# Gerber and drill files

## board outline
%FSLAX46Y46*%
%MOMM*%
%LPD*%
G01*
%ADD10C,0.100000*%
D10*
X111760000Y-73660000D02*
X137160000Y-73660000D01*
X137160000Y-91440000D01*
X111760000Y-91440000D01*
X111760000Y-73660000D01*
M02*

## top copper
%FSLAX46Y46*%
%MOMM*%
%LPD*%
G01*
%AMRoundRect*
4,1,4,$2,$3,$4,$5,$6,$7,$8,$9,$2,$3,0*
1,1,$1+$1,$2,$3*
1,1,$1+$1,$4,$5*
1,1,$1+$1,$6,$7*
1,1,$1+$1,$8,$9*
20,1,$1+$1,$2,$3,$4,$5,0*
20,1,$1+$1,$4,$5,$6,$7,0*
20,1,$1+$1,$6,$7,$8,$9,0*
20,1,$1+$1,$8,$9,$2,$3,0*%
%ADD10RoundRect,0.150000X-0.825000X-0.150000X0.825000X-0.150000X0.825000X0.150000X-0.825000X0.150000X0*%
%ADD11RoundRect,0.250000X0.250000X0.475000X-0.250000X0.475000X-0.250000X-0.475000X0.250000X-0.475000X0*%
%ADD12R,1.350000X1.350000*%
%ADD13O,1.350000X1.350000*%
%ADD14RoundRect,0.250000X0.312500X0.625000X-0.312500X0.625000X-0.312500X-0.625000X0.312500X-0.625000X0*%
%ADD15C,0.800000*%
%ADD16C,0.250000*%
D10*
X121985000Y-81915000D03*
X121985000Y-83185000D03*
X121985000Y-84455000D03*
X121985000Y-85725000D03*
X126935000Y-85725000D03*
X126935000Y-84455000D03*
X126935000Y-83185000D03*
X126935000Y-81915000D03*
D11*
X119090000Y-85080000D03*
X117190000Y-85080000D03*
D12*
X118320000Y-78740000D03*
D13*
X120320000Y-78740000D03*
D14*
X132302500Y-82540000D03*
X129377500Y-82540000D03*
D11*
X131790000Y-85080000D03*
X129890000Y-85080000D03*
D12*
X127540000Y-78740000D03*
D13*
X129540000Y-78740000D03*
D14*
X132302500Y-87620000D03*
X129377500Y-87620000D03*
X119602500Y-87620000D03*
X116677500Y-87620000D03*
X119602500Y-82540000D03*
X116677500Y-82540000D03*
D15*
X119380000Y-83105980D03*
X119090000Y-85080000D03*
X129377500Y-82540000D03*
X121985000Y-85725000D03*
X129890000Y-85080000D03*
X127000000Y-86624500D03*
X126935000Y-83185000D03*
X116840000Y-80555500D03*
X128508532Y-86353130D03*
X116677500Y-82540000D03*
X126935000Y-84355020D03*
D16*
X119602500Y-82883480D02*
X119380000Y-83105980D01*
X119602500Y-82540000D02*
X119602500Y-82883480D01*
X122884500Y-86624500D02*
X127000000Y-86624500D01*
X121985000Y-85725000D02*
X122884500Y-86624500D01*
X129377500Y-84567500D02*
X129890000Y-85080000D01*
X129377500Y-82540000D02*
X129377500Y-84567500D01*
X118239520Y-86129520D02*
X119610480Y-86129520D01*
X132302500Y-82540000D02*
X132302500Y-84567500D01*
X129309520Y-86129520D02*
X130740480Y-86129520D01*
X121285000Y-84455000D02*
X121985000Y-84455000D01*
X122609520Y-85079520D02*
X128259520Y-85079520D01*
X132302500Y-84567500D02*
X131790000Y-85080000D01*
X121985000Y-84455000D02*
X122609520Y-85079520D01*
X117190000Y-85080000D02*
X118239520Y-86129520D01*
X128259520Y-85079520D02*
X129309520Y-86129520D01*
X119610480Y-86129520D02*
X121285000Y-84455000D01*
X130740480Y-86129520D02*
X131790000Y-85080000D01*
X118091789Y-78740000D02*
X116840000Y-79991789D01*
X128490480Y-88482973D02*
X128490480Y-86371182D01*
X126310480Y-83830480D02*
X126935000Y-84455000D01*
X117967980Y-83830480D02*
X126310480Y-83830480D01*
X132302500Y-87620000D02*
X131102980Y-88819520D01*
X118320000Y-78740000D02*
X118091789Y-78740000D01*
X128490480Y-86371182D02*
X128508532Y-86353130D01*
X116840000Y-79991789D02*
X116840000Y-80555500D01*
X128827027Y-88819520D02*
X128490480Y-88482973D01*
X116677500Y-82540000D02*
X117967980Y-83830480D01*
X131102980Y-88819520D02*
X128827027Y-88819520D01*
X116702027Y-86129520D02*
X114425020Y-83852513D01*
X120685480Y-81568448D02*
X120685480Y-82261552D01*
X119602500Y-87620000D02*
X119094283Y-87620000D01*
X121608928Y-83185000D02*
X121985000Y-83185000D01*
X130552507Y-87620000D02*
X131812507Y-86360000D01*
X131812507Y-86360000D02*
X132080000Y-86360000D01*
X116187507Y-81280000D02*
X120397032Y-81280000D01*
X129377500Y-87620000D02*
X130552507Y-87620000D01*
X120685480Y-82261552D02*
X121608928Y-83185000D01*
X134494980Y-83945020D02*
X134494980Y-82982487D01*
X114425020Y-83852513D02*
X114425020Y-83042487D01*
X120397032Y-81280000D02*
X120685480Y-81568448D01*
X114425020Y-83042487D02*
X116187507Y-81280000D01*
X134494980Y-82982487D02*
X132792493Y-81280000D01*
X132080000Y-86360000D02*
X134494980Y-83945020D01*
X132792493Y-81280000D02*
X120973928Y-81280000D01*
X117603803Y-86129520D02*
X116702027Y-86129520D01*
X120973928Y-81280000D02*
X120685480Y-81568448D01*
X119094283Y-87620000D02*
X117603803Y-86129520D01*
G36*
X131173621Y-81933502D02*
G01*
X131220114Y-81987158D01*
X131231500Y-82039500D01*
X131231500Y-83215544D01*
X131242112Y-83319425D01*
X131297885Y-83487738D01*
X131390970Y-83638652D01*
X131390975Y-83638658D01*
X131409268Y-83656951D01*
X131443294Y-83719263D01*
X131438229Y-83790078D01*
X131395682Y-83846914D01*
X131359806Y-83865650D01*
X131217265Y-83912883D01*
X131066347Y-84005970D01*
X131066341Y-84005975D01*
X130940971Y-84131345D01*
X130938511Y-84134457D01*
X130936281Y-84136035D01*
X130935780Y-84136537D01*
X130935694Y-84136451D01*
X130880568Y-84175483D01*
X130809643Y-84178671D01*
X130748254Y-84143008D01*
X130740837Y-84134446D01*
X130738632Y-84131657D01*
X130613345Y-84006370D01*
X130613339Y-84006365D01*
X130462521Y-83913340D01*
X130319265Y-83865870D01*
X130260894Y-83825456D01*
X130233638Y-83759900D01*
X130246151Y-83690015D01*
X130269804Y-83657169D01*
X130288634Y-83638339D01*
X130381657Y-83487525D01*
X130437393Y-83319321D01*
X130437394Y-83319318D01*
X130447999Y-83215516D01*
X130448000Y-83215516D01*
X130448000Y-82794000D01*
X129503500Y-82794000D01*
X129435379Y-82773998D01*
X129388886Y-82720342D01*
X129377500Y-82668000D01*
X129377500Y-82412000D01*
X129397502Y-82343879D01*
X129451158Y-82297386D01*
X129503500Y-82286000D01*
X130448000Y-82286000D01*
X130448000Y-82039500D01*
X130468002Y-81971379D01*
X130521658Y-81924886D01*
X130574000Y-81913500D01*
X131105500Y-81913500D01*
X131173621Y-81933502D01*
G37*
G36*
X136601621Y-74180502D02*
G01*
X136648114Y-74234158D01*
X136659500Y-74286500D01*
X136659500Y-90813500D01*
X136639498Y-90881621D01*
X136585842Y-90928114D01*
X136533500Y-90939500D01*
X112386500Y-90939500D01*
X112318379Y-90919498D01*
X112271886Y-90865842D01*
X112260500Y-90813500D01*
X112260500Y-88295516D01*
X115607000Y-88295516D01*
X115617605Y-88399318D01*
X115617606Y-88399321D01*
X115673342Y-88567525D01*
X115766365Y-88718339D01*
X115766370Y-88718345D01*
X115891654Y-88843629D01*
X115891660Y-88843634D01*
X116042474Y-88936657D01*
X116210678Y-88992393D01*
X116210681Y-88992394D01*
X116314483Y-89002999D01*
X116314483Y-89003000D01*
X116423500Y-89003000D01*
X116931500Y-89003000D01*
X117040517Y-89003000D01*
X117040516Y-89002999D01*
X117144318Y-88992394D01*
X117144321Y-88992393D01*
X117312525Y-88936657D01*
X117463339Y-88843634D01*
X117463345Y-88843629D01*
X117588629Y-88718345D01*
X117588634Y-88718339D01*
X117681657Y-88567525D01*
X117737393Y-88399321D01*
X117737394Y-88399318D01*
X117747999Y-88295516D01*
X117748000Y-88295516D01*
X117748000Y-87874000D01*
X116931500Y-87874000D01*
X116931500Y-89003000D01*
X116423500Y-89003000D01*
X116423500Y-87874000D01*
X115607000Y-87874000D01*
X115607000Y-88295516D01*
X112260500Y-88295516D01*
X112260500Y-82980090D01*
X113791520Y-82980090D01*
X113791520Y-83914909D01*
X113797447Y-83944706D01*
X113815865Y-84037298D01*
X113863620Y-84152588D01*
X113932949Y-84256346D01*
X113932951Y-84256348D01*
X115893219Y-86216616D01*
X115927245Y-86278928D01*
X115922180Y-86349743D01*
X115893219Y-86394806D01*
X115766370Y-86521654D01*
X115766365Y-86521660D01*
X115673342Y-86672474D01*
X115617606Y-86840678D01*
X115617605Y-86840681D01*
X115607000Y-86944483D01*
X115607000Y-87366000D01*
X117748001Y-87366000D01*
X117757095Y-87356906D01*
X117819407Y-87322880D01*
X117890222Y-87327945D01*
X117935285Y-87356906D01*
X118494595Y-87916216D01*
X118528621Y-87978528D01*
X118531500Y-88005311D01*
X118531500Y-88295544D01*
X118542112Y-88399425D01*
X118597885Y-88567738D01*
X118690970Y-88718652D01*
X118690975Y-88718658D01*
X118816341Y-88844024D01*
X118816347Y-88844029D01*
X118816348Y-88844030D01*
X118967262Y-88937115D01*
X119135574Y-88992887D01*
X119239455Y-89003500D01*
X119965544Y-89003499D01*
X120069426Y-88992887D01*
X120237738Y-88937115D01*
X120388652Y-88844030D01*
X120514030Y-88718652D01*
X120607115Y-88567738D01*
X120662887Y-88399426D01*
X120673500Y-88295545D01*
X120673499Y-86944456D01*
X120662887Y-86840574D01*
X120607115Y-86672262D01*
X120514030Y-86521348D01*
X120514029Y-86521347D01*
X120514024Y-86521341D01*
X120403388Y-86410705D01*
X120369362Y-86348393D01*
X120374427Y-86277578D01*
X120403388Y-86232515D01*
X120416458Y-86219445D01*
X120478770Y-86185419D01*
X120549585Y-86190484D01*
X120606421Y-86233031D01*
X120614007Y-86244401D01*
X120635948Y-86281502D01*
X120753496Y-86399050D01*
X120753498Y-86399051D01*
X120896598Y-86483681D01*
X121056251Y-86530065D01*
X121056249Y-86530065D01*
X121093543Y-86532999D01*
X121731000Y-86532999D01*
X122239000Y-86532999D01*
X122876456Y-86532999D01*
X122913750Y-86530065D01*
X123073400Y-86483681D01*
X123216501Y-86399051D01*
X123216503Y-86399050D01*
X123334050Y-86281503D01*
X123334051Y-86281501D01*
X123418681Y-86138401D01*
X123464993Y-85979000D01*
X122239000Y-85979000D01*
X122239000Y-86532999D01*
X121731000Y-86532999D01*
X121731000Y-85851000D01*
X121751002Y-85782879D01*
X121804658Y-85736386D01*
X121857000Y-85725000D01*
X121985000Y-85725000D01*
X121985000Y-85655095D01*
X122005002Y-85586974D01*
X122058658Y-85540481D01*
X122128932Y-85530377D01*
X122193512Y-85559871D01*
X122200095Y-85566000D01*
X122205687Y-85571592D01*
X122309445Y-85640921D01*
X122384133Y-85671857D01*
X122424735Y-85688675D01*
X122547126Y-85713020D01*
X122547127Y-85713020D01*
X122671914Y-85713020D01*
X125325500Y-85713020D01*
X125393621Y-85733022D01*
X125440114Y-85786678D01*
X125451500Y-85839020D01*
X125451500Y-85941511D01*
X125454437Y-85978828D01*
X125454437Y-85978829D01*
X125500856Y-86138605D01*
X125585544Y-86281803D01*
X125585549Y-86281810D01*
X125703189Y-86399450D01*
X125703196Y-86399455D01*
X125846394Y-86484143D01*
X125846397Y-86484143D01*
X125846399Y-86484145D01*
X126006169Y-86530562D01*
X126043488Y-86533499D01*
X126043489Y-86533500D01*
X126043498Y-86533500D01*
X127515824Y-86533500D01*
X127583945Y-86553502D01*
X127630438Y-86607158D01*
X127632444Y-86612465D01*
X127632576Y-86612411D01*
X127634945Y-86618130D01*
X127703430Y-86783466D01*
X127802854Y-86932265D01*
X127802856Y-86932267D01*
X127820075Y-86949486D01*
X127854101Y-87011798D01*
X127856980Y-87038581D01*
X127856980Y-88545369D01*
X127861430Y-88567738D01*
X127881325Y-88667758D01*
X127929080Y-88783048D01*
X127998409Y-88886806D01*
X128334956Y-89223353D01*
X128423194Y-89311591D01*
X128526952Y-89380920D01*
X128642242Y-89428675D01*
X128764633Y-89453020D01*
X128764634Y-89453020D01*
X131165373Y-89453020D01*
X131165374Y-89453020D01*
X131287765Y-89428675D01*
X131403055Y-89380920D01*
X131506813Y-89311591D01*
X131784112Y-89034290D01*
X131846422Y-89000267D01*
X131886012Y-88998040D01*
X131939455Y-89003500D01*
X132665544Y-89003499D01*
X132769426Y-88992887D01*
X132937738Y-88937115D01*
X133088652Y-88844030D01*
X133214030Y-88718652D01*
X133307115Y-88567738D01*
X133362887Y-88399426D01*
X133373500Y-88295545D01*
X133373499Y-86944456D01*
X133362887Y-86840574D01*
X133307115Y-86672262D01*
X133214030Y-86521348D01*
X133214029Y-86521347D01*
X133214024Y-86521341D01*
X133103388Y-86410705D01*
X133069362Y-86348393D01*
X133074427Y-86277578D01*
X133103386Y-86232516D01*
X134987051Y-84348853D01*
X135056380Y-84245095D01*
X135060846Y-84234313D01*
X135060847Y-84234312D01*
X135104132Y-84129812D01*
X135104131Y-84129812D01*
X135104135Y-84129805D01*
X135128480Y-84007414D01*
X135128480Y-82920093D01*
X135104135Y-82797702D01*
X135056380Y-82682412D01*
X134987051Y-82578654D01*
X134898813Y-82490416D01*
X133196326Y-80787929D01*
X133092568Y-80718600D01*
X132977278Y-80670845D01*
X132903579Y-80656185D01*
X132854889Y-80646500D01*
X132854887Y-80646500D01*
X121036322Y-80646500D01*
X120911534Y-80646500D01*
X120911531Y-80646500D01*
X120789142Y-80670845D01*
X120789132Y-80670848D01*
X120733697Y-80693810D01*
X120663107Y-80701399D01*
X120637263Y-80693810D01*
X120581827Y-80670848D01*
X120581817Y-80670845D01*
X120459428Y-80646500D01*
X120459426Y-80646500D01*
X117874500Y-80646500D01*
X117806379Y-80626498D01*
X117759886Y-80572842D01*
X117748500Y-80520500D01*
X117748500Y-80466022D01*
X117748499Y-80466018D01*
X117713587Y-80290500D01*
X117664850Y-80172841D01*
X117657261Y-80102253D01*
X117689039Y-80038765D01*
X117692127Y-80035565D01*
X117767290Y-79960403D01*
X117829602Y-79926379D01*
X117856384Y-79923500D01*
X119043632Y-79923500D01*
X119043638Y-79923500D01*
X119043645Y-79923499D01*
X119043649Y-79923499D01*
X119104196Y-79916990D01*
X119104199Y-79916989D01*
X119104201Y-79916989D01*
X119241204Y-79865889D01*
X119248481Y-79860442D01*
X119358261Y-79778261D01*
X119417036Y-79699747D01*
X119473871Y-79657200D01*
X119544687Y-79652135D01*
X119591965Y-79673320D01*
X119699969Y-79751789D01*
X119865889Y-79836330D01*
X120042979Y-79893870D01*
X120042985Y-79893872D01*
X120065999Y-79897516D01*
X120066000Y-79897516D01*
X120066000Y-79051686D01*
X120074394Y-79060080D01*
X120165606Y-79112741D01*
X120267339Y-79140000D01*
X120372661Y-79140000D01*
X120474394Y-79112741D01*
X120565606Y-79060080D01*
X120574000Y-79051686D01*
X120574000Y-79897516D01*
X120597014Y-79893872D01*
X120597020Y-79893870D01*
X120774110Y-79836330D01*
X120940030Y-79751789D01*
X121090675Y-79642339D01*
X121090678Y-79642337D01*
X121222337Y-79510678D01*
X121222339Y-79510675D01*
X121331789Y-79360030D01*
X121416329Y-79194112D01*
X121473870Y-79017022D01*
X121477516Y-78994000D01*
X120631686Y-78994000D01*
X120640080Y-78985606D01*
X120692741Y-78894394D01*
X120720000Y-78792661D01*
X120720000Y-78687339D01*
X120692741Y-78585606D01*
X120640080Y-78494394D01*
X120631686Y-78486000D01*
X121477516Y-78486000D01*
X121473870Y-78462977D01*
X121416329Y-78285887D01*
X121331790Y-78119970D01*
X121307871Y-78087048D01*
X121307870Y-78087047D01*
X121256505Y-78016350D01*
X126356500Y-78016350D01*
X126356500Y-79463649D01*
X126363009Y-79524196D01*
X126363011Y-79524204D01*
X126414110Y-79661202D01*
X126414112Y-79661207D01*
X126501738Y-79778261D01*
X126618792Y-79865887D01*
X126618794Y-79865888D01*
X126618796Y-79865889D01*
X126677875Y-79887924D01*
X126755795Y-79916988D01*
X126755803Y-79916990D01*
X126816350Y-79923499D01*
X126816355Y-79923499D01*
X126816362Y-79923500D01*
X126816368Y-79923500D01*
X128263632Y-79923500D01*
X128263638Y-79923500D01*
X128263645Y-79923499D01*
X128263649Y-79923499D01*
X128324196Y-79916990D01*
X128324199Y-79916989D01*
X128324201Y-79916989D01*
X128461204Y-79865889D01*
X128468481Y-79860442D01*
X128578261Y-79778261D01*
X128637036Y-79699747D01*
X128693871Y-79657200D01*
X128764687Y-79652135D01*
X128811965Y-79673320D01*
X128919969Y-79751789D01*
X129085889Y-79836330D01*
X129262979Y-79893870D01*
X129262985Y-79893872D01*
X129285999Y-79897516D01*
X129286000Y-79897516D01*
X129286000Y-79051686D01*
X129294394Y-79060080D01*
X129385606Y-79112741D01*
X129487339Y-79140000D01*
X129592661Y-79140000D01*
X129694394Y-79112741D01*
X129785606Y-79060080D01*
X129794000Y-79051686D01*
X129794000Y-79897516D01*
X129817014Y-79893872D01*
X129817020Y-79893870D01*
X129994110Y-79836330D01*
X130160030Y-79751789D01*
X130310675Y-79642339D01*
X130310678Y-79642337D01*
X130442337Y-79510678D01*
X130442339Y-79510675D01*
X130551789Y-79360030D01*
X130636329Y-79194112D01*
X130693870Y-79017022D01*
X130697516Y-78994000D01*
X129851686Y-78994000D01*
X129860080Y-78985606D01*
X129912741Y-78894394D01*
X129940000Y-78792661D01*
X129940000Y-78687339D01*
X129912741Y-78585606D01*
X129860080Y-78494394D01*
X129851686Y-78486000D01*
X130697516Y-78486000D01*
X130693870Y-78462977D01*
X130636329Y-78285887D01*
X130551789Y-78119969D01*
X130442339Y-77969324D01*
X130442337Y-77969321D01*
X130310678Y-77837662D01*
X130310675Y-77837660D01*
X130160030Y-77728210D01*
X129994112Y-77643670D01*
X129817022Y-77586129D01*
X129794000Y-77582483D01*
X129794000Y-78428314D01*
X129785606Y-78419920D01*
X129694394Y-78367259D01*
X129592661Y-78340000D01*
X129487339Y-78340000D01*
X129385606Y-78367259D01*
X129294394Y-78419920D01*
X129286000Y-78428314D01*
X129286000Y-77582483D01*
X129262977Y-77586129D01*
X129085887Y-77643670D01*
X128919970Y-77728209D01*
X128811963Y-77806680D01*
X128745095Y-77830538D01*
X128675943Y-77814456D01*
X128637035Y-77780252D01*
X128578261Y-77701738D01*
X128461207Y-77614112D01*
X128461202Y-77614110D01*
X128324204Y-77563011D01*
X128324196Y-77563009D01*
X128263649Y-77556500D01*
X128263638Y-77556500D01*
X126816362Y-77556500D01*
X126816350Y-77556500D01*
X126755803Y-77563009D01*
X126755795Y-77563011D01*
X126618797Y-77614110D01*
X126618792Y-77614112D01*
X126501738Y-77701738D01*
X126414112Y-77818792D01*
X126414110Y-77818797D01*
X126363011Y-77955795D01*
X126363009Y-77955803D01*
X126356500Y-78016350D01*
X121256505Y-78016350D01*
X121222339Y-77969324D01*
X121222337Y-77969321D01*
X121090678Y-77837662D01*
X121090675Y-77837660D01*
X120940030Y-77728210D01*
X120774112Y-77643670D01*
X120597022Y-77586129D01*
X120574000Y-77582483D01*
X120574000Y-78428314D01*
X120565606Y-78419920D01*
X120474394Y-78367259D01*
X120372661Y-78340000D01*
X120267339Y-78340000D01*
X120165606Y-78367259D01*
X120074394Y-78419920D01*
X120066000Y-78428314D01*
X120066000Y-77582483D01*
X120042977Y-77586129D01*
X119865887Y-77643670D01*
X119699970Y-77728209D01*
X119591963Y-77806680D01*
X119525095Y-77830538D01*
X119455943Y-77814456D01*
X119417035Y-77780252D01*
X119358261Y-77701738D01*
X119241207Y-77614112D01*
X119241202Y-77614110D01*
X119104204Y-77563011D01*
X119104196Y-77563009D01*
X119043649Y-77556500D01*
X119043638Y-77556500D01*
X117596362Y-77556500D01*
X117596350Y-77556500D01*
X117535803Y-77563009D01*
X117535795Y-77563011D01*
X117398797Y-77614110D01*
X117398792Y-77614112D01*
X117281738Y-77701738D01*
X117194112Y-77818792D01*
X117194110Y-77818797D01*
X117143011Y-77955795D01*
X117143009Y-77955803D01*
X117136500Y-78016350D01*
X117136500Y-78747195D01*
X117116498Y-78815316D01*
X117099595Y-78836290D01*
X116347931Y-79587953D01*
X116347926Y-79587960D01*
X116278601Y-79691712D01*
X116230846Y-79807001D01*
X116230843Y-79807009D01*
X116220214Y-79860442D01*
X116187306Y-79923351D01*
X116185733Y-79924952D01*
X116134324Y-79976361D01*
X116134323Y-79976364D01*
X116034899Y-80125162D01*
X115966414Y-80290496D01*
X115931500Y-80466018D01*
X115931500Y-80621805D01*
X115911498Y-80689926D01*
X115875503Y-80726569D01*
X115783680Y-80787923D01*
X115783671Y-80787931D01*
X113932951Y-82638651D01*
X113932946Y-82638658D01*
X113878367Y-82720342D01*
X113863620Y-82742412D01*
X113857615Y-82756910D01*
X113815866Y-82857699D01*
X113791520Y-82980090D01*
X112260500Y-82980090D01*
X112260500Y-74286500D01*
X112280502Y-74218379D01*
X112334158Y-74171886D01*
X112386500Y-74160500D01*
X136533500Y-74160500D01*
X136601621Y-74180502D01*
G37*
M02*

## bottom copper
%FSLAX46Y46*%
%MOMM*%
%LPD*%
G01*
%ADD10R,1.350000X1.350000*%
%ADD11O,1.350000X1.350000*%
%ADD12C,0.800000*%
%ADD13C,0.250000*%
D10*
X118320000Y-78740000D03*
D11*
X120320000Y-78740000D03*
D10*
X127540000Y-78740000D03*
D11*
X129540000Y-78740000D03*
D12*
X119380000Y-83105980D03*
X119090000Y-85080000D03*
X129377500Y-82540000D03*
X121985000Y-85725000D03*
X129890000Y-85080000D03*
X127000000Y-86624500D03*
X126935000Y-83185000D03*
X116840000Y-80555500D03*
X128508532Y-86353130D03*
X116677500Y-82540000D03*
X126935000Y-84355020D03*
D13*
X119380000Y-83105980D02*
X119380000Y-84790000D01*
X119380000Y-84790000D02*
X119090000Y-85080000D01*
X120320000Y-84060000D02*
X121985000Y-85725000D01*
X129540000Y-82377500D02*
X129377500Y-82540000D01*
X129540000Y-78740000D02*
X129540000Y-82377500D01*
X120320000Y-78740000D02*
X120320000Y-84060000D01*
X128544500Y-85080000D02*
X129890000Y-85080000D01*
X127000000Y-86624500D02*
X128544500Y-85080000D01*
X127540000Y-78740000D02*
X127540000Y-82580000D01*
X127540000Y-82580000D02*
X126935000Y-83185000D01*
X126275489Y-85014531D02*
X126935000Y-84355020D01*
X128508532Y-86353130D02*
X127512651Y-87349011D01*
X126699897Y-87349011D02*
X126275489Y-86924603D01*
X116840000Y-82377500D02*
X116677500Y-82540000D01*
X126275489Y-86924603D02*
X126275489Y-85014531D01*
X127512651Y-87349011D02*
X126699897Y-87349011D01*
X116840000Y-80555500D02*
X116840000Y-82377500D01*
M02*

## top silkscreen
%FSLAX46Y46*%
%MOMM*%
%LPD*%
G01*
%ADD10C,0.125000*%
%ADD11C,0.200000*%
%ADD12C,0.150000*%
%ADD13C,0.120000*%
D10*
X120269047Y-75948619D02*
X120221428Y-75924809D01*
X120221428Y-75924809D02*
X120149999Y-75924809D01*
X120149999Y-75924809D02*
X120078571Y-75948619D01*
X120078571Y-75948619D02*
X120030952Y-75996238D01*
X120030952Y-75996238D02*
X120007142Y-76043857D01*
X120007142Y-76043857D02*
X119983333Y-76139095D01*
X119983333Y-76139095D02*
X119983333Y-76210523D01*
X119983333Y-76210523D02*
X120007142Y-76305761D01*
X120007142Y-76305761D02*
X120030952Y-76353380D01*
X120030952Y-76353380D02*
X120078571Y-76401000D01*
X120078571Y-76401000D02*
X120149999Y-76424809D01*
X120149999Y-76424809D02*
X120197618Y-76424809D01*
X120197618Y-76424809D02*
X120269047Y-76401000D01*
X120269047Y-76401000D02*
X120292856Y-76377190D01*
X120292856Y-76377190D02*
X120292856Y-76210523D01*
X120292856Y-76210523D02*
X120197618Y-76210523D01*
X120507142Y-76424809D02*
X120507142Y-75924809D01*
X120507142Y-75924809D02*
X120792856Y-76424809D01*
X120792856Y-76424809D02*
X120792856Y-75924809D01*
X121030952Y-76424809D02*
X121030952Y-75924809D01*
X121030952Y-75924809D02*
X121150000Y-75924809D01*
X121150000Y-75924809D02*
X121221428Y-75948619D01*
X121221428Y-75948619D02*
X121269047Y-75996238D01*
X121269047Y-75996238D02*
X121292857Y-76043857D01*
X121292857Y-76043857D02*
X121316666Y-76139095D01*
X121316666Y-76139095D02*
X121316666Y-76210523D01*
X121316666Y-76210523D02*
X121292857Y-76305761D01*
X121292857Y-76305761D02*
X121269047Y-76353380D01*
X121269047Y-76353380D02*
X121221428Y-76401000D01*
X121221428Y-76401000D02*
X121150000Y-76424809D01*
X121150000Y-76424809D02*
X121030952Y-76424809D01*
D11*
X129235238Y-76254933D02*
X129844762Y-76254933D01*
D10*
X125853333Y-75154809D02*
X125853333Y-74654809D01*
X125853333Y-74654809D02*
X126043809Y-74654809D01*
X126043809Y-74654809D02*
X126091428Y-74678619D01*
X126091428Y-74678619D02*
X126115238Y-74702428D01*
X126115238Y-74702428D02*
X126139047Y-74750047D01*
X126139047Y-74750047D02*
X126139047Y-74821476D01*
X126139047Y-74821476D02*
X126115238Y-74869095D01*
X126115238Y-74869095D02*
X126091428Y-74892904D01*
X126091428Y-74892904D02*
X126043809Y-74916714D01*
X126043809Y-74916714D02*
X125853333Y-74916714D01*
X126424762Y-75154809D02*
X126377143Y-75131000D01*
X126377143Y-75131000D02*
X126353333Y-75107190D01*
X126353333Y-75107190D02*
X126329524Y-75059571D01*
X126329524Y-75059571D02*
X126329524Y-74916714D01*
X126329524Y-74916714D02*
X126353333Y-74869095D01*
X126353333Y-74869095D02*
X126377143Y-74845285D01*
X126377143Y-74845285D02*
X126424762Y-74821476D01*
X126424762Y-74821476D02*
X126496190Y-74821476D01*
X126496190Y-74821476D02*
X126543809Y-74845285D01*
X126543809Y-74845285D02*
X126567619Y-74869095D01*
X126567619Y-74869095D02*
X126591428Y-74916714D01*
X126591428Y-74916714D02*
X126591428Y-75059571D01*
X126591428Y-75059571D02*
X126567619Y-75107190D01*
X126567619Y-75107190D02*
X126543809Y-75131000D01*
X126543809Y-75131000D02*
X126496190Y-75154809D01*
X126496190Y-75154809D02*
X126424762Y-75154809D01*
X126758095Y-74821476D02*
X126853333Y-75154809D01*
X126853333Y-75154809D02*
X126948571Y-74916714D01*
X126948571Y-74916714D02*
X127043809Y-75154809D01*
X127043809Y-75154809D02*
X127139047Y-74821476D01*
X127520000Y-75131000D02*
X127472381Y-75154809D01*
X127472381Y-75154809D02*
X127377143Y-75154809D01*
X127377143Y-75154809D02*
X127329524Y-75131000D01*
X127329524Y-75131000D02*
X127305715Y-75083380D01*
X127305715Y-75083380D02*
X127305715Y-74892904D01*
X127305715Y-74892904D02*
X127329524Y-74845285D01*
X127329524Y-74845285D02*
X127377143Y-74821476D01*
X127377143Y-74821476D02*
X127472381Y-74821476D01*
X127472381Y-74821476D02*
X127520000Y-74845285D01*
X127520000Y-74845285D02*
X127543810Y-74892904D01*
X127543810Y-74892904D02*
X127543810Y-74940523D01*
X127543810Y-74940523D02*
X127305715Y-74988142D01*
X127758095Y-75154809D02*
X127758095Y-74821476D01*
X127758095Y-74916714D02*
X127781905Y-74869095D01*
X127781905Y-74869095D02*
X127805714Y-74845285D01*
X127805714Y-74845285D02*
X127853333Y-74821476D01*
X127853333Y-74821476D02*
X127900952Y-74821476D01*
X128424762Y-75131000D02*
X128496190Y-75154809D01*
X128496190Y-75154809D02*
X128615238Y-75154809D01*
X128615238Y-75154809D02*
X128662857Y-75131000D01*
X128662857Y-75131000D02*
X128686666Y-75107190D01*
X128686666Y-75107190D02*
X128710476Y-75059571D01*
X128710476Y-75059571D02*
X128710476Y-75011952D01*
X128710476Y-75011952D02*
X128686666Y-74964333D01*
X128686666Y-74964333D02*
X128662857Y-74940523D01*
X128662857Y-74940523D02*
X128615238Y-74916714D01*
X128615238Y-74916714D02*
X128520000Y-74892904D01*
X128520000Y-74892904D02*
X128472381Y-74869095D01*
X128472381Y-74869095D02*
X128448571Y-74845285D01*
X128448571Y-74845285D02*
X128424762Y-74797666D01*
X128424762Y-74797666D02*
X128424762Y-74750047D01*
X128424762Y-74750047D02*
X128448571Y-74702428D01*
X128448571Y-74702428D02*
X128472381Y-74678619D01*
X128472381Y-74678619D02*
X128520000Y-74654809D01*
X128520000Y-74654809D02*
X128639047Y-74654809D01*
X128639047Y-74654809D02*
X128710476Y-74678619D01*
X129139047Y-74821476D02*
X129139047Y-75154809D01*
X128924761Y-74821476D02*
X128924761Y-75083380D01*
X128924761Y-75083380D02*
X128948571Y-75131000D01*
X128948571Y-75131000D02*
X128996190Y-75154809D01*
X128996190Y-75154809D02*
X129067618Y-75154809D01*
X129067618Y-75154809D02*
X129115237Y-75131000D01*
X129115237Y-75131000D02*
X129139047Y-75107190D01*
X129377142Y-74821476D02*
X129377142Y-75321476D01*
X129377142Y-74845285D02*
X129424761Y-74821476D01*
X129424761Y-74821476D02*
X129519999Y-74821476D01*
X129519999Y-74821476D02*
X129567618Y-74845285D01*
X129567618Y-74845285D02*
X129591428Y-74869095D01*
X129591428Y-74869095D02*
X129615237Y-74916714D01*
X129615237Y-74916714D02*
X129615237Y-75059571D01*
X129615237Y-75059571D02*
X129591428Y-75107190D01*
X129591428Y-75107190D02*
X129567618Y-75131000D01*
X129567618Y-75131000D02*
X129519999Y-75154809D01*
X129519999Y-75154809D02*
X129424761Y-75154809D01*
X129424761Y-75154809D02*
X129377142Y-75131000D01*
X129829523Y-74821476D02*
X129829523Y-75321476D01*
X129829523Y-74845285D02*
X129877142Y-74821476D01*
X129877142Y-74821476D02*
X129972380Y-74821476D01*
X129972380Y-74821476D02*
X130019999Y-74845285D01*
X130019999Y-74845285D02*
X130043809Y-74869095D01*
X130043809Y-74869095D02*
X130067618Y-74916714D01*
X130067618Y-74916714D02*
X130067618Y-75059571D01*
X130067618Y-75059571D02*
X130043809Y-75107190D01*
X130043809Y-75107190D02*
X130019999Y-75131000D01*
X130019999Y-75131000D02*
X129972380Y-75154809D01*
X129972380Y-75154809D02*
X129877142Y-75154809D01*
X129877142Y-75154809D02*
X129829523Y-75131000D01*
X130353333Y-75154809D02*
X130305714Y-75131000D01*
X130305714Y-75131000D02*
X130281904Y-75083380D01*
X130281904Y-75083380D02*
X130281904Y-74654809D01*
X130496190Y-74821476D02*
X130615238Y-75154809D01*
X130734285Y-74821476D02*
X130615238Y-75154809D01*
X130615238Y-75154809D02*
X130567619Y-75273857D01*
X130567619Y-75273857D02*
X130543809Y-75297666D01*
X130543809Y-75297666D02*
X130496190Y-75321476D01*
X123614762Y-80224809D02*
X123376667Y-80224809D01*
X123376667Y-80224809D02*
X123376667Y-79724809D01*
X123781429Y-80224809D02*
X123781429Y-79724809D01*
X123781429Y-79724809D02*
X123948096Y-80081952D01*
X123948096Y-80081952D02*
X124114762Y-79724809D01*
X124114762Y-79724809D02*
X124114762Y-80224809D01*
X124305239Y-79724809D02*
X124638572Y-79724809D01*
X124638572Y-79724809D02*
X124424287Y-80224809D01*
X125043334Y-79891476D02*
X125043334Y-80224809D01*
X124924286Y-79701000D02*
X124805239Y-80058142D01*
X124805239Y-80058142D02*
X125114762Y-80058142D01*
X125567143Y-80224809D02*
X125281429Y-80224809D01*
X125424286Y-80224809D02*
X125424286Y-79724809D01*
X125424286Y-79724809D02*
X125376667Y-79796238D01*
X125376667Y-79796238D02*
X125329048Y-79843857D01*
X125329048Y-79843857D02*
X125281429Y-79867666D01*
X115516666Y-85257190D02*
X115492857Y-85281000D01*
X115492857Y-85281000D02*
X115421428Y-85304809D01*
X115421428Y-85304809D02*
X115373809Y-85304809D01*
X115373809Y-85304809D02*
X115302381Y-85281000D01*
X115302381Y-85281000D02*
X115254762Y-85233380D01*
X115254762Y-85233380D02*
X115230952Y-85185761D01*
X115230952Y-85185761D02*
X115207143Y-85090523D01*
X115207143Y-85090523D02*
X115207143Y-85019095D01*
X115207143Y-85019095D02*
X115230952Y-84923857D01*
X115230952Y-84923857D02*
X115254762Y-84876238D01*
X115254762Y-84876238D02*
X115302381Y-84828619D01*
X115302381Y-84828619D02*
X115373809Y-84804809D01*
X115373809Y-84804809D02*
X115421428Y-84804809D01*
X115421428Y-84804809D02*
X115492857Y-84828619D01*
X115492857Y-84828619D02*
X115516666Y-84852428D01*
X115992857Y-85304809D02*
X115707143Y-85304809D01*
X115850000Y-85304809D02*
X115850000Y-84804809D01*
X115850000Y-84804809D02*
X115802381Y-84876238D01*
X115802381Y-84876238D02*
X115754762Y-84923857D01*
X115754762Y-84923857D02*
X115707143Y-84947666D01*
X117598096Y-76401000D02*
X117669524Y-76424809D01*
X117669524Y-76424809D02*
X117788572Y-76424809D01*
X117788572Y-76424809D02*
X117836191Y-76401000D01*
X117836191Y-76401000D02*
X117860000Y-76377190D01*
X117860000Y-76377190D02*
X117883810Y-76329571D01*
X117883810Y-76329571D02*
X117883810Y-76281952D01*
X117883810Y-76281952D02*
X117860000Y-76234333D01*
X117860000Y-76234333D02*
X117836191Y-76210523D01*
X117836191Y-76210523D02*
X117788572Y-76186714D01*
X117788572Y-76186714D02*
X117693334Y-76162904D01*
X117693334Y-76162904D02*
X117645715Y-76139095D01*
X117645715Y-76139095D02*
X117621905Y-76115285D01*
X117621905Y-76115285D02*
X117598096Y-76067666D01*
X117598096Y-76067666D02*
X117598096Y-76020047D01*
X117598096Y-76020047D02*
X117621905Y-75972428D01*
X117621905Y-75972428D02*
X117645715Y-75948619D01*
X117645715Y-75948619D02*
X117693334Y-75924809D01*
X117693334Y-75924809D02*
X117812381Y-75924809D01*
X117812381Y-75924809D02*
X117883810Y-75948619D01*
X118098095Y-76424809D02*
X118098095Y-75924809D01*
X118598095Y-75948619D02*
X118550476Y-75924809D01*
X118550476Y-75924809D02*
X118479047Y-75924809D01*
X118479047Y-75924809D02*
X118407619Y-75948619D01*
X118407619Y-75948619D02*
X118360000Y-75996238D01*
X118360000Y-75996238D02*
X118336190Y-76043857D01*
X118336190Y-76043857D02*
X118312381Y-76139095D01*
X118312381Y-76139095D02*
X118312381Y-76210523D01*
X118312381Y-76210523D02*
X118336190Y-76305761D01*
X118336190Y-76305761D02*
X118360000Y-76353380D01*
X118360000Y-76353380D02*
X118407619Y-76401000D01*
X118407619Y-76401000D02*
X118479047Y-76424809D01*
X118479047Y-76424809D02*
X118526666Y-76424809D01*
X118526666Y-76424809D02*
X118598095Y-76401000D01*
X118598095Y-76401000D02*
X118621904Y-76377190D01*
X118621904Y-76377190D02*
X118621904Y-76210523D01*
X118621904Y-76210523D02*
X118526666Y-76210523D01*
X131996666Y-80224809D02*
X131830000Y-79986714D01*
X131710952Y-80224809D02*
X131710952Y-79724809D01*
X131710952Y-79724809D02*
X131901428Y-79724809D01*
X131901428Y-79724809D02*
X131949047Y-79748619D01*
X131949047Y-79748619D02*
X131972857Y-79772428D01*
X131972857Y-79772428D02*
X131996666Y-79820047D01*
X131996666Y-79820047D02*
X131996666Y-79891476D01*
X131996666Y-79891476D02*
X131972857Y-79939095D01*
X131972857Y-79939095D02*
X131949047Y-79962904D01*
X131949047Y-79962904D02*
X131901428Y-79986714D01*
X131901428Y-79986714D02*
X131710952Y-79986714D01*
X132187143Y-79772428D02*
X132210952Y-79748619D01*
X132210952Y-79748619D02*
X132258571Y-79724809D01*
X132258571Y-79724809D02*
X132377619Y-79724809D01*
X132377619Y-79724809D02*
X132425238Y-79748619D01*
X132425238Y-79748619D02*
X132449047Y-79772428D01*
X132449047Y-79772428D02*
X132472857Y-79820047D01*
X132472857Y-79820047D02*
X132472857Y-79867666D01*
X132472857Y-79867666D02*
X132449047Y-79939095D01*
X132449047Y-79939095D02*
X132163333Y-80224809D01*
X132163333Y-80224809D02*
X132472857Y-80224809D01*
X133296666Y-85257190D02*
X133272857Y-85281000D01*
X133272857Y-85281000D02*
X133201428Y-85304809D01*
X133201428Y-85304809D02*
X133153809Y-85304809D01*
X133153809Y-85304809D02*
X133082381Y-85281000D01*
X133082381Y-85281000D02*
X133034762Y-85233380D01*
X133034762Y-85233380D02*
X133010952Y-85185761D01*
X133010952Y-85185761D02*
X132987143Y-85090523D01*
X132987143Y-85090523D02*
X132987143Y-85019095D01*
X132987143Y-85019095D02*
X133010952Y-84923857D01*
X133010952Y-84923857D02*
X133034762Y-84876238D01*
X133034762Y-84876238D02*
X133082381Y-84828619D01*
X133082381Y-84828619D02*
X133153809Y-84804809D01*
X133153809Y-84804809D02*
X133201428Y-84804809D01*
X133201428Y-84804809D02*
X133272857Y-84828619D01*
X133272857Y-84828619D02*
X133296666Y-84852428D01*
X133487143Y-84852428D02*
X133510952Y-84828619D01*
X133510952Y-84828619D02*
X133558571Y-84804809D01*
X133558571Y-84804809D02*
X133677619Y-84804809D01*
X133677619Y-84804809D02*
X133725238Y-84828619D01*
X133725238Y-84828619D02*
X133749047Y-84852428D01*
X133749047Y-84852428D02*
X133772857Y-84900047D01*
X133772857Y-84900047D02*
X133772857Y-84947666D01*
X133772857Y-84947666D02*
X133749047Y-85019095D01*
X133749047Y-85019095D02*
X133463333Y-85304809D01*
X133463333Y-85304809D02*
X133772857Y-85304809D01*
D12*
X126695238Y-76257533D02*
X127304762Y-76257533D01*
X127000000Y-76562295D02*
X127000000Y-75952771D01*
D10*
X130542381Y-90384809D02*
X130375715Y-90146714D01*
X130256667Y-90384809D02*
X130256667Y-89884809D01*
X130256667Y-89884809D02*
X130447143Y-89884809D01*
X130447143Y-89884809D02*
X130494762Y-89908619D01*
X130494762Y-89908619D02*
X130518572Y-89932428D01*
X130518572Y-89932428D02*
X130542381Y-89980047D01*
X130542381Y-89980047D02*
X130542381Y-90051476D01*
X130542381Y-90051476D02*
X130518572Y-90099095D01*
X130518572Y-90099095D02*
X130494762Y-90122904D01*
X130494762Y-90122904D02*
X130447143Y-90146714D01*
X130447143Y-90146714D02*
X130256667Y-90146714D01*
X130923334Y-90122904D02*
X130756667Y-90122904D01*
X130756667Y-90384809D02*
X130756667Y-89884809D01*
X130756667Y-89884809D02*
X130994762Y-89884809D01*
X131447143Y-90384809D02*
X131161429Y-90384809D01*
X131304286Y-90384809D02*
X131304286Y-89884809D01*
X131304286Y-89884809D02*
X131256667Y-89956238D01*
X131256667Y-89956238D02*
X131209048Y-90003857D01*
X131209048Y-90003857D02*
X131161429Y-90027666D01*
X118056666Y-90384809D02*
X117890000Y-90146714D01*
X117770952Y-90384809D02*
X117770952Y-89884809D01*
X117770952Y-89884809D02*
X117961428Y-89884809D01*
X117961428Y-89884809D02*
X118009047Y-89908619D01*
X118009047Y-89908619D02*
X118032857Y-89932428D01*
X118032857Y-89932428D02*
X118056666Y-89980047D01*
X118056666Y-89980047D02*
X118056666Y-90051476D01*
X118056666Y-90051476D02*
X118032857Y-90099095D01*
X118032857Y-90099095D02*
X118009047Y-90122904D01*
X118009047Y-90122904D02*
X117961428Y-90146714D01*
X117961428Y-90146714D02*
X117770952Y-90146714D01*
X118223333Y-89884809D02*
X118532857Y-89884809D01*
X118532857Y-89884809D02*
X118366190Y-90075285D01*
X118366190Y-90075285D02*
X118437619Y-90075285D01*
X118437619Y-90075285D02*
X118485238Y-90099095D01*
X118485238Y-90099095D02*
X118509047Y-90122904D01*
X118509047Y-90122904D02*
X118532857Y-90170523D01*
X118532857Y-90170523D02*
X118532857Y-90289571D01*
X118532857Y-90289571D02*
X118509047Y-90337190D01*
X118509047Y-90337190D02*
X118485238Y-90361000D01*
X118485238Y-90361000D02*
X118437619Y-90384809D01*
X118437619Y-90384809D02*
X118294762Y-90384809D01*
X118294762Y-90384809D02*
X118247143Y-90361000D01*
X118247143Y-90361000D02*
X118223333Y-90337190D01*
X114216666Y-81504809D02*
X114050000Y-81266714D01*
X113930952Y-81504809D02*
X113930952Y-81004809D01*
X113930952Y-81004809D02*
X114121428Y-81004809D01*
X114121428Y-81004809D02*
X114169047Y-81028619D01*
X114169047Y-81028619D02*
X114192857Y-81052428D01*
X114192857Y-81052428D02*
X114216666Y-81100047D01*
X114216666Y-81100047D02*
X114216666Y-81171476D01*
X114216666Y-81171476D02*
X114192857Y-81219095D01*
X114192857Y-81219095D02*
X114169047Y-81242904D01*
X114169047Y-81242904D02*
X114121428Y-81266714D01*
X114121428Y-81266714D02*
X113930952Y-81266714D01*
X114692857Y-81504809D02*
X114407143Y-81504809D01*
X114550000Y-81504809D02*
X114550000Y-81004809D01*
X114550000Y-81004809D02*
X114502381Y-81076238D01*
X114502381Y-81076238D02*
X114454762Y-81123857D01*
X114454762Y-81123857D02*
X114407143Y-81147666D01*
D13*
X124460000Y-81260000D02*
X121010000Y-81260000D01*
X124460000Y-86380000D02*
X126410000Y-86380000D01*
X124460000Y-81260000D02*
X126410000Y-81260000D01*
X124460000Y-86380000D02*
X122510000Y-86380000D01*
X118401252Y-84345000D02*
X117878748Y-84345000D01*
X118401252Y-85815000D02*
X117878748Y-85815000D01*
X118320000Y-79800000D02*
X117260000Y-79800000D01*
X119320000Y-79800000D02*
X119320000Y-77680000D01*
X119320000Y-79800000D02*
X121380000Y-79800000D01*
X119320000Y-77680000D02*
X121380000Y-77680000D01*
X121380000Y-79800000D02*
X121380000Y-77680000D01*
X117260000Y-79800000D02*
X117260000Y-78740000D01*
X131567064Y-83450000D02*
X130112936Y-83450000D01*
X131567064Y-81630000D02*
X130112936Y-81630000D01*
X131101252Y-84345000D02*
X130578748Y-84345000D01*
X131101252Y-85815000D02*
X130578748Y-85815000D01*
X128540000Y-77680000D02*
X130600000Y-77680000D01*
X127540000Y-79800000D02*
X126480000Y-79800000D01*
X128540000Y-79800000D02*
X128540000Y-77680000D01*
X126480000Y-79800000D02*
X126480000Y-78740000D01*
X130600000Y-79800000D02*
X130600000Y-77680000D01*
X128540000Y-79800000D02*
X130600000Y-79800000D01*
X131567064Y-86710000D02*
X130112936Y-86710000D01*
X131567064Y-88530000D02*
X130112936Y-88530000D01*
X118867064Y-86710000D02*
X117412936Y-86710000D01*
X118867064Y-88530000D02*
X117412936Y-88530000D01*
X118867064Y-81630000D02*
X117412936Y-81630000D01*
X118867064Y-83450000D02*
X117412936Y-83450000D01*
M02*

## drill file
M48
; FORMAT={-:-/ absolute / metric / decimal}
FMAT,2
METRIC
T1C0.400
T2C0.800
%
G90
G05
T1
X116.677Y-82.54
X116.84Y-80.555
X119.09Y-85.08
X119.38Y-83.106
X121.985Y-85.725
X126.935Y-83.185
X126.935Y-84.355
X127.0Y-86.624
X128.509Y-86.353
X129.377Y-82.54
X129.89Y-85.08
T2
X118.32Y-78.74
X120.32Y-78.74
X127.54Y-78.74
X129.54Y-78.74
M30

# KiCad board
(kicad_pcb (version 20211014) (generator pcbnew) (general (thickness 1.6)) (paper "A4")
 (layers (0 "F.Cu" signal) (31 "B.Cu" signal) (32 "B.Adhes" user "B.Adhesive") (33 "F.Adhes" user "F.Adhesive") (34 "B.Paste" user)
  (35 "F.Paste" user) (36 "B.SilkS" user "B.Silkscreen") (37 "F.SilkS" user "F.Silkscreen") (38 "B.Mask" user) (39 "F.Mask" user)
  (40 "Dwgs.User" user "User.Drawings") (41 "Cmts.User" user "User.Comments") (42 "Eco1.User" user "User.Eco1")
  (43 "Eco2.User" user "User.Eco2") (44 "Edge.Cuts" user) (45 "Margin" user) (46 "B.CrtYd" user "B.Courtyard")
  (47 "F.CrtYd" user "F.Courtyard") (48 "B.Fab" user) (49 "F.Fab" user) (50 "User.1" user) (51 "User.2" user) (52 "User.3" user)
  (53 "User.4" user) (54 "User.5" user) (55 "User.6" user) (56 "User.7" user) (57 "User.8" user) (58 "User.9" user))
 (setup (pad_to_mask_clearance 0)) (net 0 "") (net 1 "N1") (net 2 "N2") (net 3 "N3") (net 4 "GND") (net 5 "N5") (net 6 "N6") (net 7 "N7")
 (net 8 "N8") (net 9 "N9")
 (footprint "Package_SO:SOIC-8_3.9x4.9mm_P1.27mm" (layer "F.Cu") (at 124.46 83.82)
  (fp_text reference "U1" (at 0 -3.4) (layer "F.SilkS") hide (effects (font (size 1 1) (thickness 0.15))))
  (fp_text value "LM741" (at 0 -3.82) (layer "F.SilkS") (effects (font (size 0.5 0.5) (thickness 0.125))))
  (fp_line (start 0 -2.56) (end -3.45 -2.56) (layer "F.SilkS") (width 0.12))
  (fp_line (start 0 2.56) (end 1.95 2.56) (layer "F.SilkS") (width 0.12))
  (fp_line (start 0 -2.56) (end 1.95 -2.56) (layer "F.SilkS") (width 0.12))
  (fp_line (start 0 2.56) (end -1.95 2.56) (layer "F.SilkS") (width 0.12))
  (pad "1" smd roundrect (at -2.475 -1.905) (size 1.95 0.6) (layers "F.Cu" "F.Paste" "F.Mask") (roundrect_rratio 0.25) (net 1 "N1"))
  (pad "2" smd roundrect (at -2.475 -0.635) (size 1.95 0.6) (layers "F.Cu" "F.Paste" "F.Mask") (roundrect_rratio 0.25) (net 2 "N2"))
  (pad "3" smd roundrect (at -2.475 0.635) (size 1.95 0.6) (layers "F.Cu" "F.Paste" "F.Mask") (roundrect_rratio 0.25) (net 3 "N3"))
  (pad "4" smd roundrect (at -2.475 1.905) (size 1.95 0.6) (layers "F.Cu" "F.Paste" "F.Mask") (roundrect_rratio 0.25) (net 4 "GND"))
  (pad "5" smd roundrect (at 2.475 1.905) (size 1.95 0.6) (layers "F.Cu" "F.Paste" "F.Mask") (roundrect_rratio 0.25) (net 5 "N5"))
  (pad "6" smd roundrect (at 2.475 0.635) (size 1.95 0.6) (layers "F.Cu" "F.Paste" "F.Mask") (roundrect_rratio 0.25) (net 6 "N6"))
  (pad "7" smd roundrect (at 2.475 -0.635) (size 1.95 0.6) (layers "F.Cu" "F.Paste" "F.Mask") (roundrect_rratio 0.25) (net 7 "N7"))
  (pad "8" smd roundrect (at 2.475 -1.905) (size 1.95 0.6) (layers "F.Cu" "F.Paste" "F.Mask") (roundrect_rratio 0.25) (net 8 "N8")))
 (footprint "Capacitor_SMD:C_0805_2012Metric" (layer "F.Cu") (at 118.14 85.08 180)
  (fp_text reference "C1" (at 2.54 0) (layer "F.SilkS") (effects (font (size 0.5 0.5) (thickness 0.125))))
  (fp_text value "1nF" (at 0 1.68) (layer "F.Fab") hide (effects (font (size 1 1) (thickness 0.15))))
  (fp_line (start -0.261252 0.735) (end 0.261252 0.735) (layer "F.SilkS") (width 0.12))
  (fp_line (start -0.261252 -0.735) (end 0.261252 -0.735) (layer "F.SilkS") (width 0.12))
  (pad "1" smd roundrect (at -0.95 0 180) (size 1 1.45) (layers "F.Cu" "F.Paste" "F.Mask") (roundrect_rratio 0.25) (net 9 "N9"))
  (pad "2" smd roundrect (at 0.95 0 180) (size 1 1.45) (layers "F.Cu" "F.Paste" "F.Mask") (roundrect_rratio 0.25) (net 3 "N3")))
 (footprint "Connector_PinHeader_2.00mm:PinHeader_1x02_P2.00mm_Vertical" (layer "F.Cu") (at 118.32 78.74 90)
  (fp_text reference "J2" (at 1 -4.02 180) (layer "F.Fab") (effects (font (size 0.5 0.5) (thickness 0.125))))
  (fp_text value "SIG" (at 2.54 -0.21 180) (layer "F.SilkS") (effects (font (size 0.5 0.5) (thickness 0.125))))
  (fp_line (start -1.06 0) (end -1.06 -1.06) (layer "F.SilkS") (width 0.12))
  (fp_line (start -1.06 1) (end 1.06 1) (layer "F.SilkS") (width 0.12))
  (fp_line (start -1.06 1) (end -1.06 3.06) (layer "F.SilkS") (width 0.12))
  (fp_line (start 1.06 1) (end 1.06 3.06) (layer "F.SilkS") (width 0.12))
  (fp_line (start -1.06 3.06) (end 1.06 3.06) (layer "F.SilkS") (width 0.12))
  (fp_line (start -1.06 -1.06) (end 0 -1.06) (layer "F.SilkS") (width 0.12))
  (pad "1" thru_hole rect (at 0 0 90) (size 1.35 1.35) (drill 0.8) (layers *.Cu *.Mask) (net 6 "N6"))
  (pad "2" thru_hole oval (at 0 2 90) (size 1.35 1.35) (drill 0.8) (layers *.Cu *.Mask) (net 4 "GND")))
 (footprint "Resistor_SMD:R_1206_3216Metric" (layer "F.Cu") (at 130.84 82.54 180)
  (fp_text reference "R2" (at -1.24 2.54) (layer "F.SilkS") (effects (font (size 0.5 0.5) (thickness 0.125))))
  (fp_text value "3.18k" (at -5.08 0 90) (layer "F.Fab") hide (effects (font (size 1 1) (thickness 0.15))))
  (fp_line (start -0.727064 -0.91) (end 0.727064 -0.91) (layer "F.SilkS") (width 0.12))
  (fp_line (start -0.727064 0.91) (end 0.727064 0.91) (layer "F.SilkS") (width 0.12))
  (pad "1" smd roundrect (at -1.4625 0 180) (size 1.125 1.75) (layers "F.Cu" "F.Paste" "F.Mask") (roundrect_rratio 0.2222222222)
   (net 3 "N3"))
  (pad "2" smd roundrect (at 1.4625 0 180) (size 1.125 1.75) (layers "F.Cu" "F.Paste" "F.Mask") (roundrect_rratio 0.2222222222)
   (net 4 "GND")))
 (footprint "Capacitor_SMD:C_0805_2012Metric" (layer "F.Cu") (at 130.84 85.08 180)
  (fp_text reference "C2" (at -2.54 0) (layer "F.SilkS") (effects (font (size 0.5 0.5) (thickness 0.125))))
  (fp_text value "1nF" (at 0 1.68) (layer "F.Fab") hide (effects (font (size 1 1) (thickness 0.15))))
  (fp_line (start -0.261252 0.735) (end 0.261252 0.735) (layer "F.SilkS") (width 0.12))
  (fp_line (start -0.261252 -0.735) (end 0.261252 -0.735) (layer "F.SilkS") (width 0.12))
  (pad "1" smd roundrect (at -0.95 0 180) (size 1 1.45) (layers "F.Cu" "F.Paste" "F.Mask") (roundrect_rratio 0.25) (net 3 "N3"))
  (pad "2" smd roundrect (at 0.95 0 180) (size 1 1.45) (layers "F.Cu" "F.Paste" "F.Mask") (roundrect_rratio 0.25) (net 4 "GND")))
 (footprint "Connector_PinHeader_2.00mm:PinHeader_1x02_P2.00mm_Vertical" (layer "F.Cu") (at 127.54 78.74 90)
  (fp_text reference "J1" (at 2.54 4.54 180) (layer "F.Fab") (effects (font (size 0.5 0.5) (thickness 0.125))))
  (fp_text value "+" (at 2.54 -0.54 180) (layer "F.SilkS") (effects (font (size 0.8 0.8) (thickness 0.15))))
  (fp_line (start 1.06 1) (end 1.06 3.06) (layer "F.SilkS") (width 0.12))
  (fp_line (start -1.06 0) (end -1.06 -1.06) (layer "F.SilkS") (width 0.12))
  (fp_line (start -1.06 1) (end 1.06 1) (layer "F.SilkS") (width 0.12))
  (fp_line (start -1.06 -1.06) (end 0 -1.06) (layer "F.SilkS") (width 0.12))
  (fp_line (start -1.06 3.06) (end 1.06 3.06) (layer "F.SilkS") (width 0.12))
  (fp_line (start -1.06 1) (end -1.06 3.06) (layer "F.SilkS") (width 0.12))
  (pad "1" thru_hole rect (at 0 0 90) (size 1.35 1.35) (drill 0.8) (layers *.Cu *.Mask) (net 7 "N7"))
  (pad "2" thru_hole oval (at 0 2 90) (size 1.35 1.35) (drill 0.8) (layers *.Cu *.Mask) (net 4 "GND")))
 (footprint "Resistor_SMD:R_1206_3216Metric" (layer "F.Cu") (at 130.84 87.62 180)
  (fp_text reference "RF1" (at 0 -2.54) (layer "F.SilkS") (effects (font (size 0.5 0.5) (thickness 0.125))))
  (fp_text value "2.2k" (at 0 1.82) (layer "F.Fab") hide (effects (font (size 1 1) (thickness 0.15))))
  (fp_line (start -0.727064 0.91) (end 0.727064 0.91) (layer "F.SilkS") (width 0.12))
  (fp_line (start -0.727064 -0.91) (end 0.727064 -0.91) (layer "F.SilkS") (width 0.12))
  (pad "1" smd roundrect (at -1.4625 0 180) (size 1.125 1.75) (layers "F.Cu" "F.Paste" "F.Mask") (roundrect_rratio 0.2222222222)
   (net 6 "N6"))
  (pad "2" smd roundrect (at 1.4625 0 180) (size 1.125 1.75) (layers "F.Cu" "F.Paste" "F.Mask") (roundrect_rratio 0.2222222222) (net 2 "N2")))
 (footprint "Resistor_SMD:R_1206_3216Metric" (layer "F.Cu") (at 118.14 87.62 180)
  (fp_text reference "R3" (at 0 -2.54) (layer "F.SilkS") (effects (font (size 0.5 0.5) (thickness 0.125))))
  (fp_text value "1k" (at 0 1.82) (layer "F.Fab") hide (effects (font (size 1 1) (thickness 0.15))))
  (fp_line (start -0.727064 0.91) (end 0.727064 0.91) (layer "F.SilkS") (width 0.12))
  (fp_line (start -0.727064 -0.91) (end 0.727064 -0.91) (layer "F.SilkS") (width 0.12))
  (pad "1" smd roundrect (at -1.4625 0 180) (size 1.125 1.75) (layers "F.Cu" "F.Paste" "F.Mask") (roundrect_rratio 0.2222222222)
   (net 2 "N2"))
  (pad "2" smd roundrect (at 1.4625 0 180) (size 1.125 1.75) (layers "F.Cu" "F.Paste" "F.Mask") (roundrect_rratio 0.2222222222)
   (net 4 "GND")))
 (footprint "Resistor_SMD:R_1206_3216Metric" (layer "F.Cu") (at 118.14 82.54 180)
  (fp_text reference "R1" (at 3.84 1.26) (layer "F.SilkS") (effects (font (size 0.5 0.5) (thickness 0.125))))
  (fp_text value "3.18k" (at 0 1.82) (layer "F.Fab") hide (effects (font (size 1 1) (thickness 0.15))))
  (fp_line (start -0.727064 0.91) (end 0.727064 0.91) (layer "F.SilkS") (width 0.12))
  (fp_line (start -0.727064 -0.91) (end 0.727064 -0.91) (layer "F.SilkS") (width 0.12))
  (pad "1" smd roundrect (at -1.4625 0 180) (size 1.125 1.75) (layers "F.Cu" "F.Paste" "F.Mask") (roundrect_rratio 0.2222222222)
   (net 9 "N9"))
  (pad "2" smd roundrect (at 1.4625 0 180) (size 1.125 1.75) (layers "F.Cu" "F.Paste" "F.Mask") (roundrect_rratio 0.2222222222) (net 6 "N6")))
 (gr_rect (start 111.76 73.66) (end 137.16 91.44) (layer "Edge.Cuts") (width 0.1) (fill none))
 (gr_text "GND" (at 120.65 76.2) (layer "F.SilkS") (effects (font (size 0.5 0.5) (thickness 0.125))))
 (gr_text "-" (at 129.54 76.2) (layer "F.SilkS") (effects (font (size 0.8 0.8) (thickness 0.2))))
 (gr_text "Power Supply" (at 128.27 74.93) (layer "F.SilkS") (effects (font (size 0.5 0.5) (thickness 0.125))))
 (segment (start 119.6025 82.88348) (end 119.38 83.10598) (width 0.25) (layer "F.Cu") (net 9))
 (segment (start 119.6025 82.54) (end 119.6025 82.88348) (width 0.25) (layer "F.Cu") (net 9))
 (via (at 119.38 83.10598) (size 0.8) (drill 0.4) (layers "F.Cu" "B.Cu") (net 9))
 (via (at 119.09 85.08) (size 0.8) (drill 0.4) (layers "F.Cu" "B.Cu") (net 9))
 (segment (start 119.38 83.10598) (end 119.38 84.79) (width 0.25) (layer "B.Cu") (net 9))
 (segment (start 119.38 84.79) (end 119.09 85.08) (width 0.25) (layer "B.Cu") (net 9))
 (segment (start 122.8845 86.6245) (end 127 86.6245) (width 0.25) (layer "F.Cu") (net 4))
 (segment (start 121.985 85.725) (end 122.8845 86.6245) (width 0.25) (layer "F.Cu") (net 4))
 (segment (start 129.3775 84.5675) (end 129.89 85.08) (width 0.25) (layer "F.Cu") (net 4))
 (segment (start 129.3775 82.54) (end 129.3775 84.5675) (width 0.25) (layer "F.Cu") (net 4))
 (via (at 129.3775 82.54) (size 0.8) (drill 0.4) (layers "F.Cu" "B.Cu") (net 4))
 (via (at 121.985 85.725) (size 0.8) (drill 0.4) (layers "F.Cu" "B.Cu") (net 4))
 (via (at 129.89 85.08) (size 0.8) (drill 0.4) (layers "F.Cu" "B.Cu") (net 4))
 (via (at 127 86.6245) (size 0.8) (drill 0.4) (layers "F.Cu" "B.Cu") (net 4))
 (segment (start 120.32 84.06) (end 121.985 85.725) (width 0.25) (layer "B.Cu") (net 4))
 (segment (start 129.54 82.3775) (end 129.3775 82.54) (width 0.25) (layer "B.Cu") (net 4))
 (segment (start 129.54 78.74) (end 129.54 82.3775) (width 0.25) (layer "B.Cu") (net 4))
 (segment (start 120.32 78.74) (end 120.32 84.06) (width 0.25) (layer "B.Cu") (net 4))
 (segment (start 128.5445 85.08) (end 129.89 85.08) (width 0.25) (layer "B.Cu") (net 4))
 (segment (start 127 86.6245) (end 128.5445 85.08) (width 0.25) (layer "B.Cu") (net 4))
 (via (at 126.935 83.185) (size 0.8) (drill 0.4) (layers "F.Cu" "B.Cu") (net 7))
 (segment (start 127.54 78.74) (end 127.54 82.58) (width 0.25) (layer "B.Cu") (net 7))
 (segment (start 127.54 82.58) (end 126.935 83.185) (width 0.25) (layer "B.Cu") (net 7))
 (segment (start 118.23952 86.12952) (end 119.61048 86.12952) (width 0.25) (layer "F.Cu") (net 3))
 (segment (start 132.3025 82.54) (end 132.3025 84.5675) (width 0.25) (layer "F.Cu") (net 3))
 (segment (start 129.30952 86.12952) (end 130.74048 86.12952) (width 0.25) (layer "F.Cu") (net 3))
 (segment (start 121.285 84.455) (end 121.985 84.455) (width 0.25) (layer "F.Cu") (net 3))
 (segment (start 122.60952 85.07952) (end 128.25952 85.07952) (width 0.25) (layer "F.Cu") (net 3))
 (segment (start 132.3025 84.5675) (end 131.79 85.08) (width 0.25) (layer "F.Cu") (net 3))
 (segment (start 121.985 84.455) (end 122.60952 85.07952) (width 0.25) (layer "F.Cu") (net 3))
 (segment (start 117.19 85.08) (end 118.23952 86.12952) (width 0.25) (layer "F.Cu") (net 3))
 (segment (start 128.25952 85.07952) (end 129.30952 86.12952) (width 0.25) (layer "F.Cu") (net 3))
 (segment (start 119.61048 86.12952) (end 121.285 84.455) (width 0.25) (layer "F.Cu") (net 3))
 (segment (start 130.74048 86.12952) (end 131.79 85.08) (width 0.25) (layer "F.Cu") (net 3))
 (segment (start 118.091789 78.74) (end 116.84 79.991789) (width 0.25) (layer "F.Cu") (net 6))
 (segment (start 128.49048 88.482973) (end 128.49048 86.371182) (width 0.25) (layer "F.Cu") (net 6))
 (segment (start 126.31048 83.83048) (end 126.935 84.455) (width 0.25) (layer "F.Cu") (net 6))
 (segment (start 117.96798 83.83048) (end 126.31048 83.83048) (width 0.25) (layer "F.Cu") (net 6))
 (segment (start 132.3025 87.62) (end 131.10298 88.81952) (width 0.25) (layer "F.Cu") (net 6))
 (segment (start 118.32 78.74) (end 118.091789 78.74) (width 0.25) (layer "F.Cu") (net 6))
 (segment (start 128.49048 86.371182) (end 128.508532 86.35313) (width 0.25) (layer "F.Cu") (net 6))
 (segment (start 116.84 79.991789) (end 116.84 80.5555) (width 0.25) (layer "F.Cu") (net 6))
 (segment (start 128.827027 88.81952) (end 128.49048 88.482973) (width 0.25) (layer "F.Cu") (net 6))
 (segment (start 116.6775 82.54) (end 117.96798 83.83048) (width 0.25) (layer "F.Cu") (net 6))
 (segment (start 131.10298 88.81952) (end 128.827027 88.81952) (width 0.25) (layer "F.Cu") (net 6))
 (via (at 116.84 80.5555) (size 0.8) (drill 0.4) (layers "F.Cu" "B.Cu") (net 6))
 (via (at 128.508532 86.35313) (size 0.8) (drill 0.4) (layers "F.Cu" "B.Cu") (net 6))
 (via (at 116.6775 82.54) (size 0.8) (drill 0.4) (layers "F.Cu" "B.Cu") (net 6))
 (via (at 126.935 84.35502) (size 0.8) (drill 0.4) (layers "F.Cu" "B.Cu") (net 6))
 (segment (start 126.275489 85.014531) (end 126.935 84.35502) (width 0.25) (layer "B.Cu") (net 6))
 (segment (start 128.508532 86.35313) (end 127.512651 87.349011) (width 0.25) (layer "B.Cu") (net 6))
 (segment (start 126.699897 87.349011) (end 126.275489 86.924603) (width 0.25) (layer "B.Cu") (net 6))
 (segment (start 116.84 82.3775) (end 116.6775 82.54) (width 0.25) (layer "B.Cu") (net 6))
 (segment (start 126.275489 86.924603) (end 126.275489 85.014531) (width 0.25) (layer "B.Cu") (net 6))
 (segment (start 127.512651 87.349011) (end 126.699897 87.349011) (width 0.25) (layer "B.Cu") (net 6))
 (segment (start 116.84 80.5555) (end 116.84 82.3775) (width 0.25) (layer "B.Cu") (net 6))
 (segment (start 116.702027 86.12952) (end 114.42502 83.852513) (width 0.25) (layer "F.Cu") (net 2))
 (segment (start 120.68548 81.568448) (end 120.68548 82.261552) (width 0.25) (layer "F.Cu") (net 2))
 (segment (start 119.6025 87.62) (end 119.094283 87.62) (width 0.25) (layer "F.Cu") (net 2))
 (segment (start 121.608928 83.185) (end 121.985 83.185) (width 0.25) (layer "F.Cu") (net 2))
 (segment (start 130.552507 87.62) (end 131.812507 86.36) (width 0.25) (layer "F.Cu") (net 2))
 (segment (start 131.812507 86.36) (end 132.08 86.36) (width 0.25) (layer "F.Cu") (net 2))
 (segment (start 116.187507 81.28) (end 120.397032 81.28) (width 0.25) (layer "F.Cu") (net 2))
 (segment (start 129.3775 87.62) (end 130.552507 87.62) (width 0.25) (layer "F.Cu") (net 2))
 (segment (start 120.68548 82.261552) (end 121.608928 83.185) (width 0.25) (layer "F.Cu") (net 2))
 (segment (start 134.49498 83.94502) (end 134.49498 82.982487) (width 0.25) (layer "F.Cu") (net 2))
 (segment (start 114.42502 83.852513) (end 114.42502 83.042487) (width 0.25) (layer "F.Cu") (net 2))
 (segment (start 120.397032 81.28) (end 120.68548 81.568448) (width 0.25) (layer "F.Cu") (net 2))
 (segment (start 114.42502 83.042487) (end 116.187507 81.28) (width 0.25) (layer "F.Cu") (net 2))
 (segment (start 134.49498 82.982487) (end 132.792493 81.28) (width 0.25) (layer "F.Cu") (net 2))
 (segment (start 132.08 86.36) (end 134.49498 83.94502) (width 0.25) (layer "F.Cu") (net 2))
 (segment (start 132.792493 81.28) (end 120.973928 81.28) (width 0.25) (layer "F.Cu") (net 2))
 (segment (start 117.603803 86.12952) (end 116.702027 86.12952) (width 0.25) (layer "F.Cu") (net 2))
 (segment (start 120.973928 81.28) (end 120.68548 81.568448) (width 0.25) (layer "F.Cu") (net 2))
 (segment (start 119.094283 87.62) (end 117.603803 86.12952) (width 0.25) (layer "F.Cu") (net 2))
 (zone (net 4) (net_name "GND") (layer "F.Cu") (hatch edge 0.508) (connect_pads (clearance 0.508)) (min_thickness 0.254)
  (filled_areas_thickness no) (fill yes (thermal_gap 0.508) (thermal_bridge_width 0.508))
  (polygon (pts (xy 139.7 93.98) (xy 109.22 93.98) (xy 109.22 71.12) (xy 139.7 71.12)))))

